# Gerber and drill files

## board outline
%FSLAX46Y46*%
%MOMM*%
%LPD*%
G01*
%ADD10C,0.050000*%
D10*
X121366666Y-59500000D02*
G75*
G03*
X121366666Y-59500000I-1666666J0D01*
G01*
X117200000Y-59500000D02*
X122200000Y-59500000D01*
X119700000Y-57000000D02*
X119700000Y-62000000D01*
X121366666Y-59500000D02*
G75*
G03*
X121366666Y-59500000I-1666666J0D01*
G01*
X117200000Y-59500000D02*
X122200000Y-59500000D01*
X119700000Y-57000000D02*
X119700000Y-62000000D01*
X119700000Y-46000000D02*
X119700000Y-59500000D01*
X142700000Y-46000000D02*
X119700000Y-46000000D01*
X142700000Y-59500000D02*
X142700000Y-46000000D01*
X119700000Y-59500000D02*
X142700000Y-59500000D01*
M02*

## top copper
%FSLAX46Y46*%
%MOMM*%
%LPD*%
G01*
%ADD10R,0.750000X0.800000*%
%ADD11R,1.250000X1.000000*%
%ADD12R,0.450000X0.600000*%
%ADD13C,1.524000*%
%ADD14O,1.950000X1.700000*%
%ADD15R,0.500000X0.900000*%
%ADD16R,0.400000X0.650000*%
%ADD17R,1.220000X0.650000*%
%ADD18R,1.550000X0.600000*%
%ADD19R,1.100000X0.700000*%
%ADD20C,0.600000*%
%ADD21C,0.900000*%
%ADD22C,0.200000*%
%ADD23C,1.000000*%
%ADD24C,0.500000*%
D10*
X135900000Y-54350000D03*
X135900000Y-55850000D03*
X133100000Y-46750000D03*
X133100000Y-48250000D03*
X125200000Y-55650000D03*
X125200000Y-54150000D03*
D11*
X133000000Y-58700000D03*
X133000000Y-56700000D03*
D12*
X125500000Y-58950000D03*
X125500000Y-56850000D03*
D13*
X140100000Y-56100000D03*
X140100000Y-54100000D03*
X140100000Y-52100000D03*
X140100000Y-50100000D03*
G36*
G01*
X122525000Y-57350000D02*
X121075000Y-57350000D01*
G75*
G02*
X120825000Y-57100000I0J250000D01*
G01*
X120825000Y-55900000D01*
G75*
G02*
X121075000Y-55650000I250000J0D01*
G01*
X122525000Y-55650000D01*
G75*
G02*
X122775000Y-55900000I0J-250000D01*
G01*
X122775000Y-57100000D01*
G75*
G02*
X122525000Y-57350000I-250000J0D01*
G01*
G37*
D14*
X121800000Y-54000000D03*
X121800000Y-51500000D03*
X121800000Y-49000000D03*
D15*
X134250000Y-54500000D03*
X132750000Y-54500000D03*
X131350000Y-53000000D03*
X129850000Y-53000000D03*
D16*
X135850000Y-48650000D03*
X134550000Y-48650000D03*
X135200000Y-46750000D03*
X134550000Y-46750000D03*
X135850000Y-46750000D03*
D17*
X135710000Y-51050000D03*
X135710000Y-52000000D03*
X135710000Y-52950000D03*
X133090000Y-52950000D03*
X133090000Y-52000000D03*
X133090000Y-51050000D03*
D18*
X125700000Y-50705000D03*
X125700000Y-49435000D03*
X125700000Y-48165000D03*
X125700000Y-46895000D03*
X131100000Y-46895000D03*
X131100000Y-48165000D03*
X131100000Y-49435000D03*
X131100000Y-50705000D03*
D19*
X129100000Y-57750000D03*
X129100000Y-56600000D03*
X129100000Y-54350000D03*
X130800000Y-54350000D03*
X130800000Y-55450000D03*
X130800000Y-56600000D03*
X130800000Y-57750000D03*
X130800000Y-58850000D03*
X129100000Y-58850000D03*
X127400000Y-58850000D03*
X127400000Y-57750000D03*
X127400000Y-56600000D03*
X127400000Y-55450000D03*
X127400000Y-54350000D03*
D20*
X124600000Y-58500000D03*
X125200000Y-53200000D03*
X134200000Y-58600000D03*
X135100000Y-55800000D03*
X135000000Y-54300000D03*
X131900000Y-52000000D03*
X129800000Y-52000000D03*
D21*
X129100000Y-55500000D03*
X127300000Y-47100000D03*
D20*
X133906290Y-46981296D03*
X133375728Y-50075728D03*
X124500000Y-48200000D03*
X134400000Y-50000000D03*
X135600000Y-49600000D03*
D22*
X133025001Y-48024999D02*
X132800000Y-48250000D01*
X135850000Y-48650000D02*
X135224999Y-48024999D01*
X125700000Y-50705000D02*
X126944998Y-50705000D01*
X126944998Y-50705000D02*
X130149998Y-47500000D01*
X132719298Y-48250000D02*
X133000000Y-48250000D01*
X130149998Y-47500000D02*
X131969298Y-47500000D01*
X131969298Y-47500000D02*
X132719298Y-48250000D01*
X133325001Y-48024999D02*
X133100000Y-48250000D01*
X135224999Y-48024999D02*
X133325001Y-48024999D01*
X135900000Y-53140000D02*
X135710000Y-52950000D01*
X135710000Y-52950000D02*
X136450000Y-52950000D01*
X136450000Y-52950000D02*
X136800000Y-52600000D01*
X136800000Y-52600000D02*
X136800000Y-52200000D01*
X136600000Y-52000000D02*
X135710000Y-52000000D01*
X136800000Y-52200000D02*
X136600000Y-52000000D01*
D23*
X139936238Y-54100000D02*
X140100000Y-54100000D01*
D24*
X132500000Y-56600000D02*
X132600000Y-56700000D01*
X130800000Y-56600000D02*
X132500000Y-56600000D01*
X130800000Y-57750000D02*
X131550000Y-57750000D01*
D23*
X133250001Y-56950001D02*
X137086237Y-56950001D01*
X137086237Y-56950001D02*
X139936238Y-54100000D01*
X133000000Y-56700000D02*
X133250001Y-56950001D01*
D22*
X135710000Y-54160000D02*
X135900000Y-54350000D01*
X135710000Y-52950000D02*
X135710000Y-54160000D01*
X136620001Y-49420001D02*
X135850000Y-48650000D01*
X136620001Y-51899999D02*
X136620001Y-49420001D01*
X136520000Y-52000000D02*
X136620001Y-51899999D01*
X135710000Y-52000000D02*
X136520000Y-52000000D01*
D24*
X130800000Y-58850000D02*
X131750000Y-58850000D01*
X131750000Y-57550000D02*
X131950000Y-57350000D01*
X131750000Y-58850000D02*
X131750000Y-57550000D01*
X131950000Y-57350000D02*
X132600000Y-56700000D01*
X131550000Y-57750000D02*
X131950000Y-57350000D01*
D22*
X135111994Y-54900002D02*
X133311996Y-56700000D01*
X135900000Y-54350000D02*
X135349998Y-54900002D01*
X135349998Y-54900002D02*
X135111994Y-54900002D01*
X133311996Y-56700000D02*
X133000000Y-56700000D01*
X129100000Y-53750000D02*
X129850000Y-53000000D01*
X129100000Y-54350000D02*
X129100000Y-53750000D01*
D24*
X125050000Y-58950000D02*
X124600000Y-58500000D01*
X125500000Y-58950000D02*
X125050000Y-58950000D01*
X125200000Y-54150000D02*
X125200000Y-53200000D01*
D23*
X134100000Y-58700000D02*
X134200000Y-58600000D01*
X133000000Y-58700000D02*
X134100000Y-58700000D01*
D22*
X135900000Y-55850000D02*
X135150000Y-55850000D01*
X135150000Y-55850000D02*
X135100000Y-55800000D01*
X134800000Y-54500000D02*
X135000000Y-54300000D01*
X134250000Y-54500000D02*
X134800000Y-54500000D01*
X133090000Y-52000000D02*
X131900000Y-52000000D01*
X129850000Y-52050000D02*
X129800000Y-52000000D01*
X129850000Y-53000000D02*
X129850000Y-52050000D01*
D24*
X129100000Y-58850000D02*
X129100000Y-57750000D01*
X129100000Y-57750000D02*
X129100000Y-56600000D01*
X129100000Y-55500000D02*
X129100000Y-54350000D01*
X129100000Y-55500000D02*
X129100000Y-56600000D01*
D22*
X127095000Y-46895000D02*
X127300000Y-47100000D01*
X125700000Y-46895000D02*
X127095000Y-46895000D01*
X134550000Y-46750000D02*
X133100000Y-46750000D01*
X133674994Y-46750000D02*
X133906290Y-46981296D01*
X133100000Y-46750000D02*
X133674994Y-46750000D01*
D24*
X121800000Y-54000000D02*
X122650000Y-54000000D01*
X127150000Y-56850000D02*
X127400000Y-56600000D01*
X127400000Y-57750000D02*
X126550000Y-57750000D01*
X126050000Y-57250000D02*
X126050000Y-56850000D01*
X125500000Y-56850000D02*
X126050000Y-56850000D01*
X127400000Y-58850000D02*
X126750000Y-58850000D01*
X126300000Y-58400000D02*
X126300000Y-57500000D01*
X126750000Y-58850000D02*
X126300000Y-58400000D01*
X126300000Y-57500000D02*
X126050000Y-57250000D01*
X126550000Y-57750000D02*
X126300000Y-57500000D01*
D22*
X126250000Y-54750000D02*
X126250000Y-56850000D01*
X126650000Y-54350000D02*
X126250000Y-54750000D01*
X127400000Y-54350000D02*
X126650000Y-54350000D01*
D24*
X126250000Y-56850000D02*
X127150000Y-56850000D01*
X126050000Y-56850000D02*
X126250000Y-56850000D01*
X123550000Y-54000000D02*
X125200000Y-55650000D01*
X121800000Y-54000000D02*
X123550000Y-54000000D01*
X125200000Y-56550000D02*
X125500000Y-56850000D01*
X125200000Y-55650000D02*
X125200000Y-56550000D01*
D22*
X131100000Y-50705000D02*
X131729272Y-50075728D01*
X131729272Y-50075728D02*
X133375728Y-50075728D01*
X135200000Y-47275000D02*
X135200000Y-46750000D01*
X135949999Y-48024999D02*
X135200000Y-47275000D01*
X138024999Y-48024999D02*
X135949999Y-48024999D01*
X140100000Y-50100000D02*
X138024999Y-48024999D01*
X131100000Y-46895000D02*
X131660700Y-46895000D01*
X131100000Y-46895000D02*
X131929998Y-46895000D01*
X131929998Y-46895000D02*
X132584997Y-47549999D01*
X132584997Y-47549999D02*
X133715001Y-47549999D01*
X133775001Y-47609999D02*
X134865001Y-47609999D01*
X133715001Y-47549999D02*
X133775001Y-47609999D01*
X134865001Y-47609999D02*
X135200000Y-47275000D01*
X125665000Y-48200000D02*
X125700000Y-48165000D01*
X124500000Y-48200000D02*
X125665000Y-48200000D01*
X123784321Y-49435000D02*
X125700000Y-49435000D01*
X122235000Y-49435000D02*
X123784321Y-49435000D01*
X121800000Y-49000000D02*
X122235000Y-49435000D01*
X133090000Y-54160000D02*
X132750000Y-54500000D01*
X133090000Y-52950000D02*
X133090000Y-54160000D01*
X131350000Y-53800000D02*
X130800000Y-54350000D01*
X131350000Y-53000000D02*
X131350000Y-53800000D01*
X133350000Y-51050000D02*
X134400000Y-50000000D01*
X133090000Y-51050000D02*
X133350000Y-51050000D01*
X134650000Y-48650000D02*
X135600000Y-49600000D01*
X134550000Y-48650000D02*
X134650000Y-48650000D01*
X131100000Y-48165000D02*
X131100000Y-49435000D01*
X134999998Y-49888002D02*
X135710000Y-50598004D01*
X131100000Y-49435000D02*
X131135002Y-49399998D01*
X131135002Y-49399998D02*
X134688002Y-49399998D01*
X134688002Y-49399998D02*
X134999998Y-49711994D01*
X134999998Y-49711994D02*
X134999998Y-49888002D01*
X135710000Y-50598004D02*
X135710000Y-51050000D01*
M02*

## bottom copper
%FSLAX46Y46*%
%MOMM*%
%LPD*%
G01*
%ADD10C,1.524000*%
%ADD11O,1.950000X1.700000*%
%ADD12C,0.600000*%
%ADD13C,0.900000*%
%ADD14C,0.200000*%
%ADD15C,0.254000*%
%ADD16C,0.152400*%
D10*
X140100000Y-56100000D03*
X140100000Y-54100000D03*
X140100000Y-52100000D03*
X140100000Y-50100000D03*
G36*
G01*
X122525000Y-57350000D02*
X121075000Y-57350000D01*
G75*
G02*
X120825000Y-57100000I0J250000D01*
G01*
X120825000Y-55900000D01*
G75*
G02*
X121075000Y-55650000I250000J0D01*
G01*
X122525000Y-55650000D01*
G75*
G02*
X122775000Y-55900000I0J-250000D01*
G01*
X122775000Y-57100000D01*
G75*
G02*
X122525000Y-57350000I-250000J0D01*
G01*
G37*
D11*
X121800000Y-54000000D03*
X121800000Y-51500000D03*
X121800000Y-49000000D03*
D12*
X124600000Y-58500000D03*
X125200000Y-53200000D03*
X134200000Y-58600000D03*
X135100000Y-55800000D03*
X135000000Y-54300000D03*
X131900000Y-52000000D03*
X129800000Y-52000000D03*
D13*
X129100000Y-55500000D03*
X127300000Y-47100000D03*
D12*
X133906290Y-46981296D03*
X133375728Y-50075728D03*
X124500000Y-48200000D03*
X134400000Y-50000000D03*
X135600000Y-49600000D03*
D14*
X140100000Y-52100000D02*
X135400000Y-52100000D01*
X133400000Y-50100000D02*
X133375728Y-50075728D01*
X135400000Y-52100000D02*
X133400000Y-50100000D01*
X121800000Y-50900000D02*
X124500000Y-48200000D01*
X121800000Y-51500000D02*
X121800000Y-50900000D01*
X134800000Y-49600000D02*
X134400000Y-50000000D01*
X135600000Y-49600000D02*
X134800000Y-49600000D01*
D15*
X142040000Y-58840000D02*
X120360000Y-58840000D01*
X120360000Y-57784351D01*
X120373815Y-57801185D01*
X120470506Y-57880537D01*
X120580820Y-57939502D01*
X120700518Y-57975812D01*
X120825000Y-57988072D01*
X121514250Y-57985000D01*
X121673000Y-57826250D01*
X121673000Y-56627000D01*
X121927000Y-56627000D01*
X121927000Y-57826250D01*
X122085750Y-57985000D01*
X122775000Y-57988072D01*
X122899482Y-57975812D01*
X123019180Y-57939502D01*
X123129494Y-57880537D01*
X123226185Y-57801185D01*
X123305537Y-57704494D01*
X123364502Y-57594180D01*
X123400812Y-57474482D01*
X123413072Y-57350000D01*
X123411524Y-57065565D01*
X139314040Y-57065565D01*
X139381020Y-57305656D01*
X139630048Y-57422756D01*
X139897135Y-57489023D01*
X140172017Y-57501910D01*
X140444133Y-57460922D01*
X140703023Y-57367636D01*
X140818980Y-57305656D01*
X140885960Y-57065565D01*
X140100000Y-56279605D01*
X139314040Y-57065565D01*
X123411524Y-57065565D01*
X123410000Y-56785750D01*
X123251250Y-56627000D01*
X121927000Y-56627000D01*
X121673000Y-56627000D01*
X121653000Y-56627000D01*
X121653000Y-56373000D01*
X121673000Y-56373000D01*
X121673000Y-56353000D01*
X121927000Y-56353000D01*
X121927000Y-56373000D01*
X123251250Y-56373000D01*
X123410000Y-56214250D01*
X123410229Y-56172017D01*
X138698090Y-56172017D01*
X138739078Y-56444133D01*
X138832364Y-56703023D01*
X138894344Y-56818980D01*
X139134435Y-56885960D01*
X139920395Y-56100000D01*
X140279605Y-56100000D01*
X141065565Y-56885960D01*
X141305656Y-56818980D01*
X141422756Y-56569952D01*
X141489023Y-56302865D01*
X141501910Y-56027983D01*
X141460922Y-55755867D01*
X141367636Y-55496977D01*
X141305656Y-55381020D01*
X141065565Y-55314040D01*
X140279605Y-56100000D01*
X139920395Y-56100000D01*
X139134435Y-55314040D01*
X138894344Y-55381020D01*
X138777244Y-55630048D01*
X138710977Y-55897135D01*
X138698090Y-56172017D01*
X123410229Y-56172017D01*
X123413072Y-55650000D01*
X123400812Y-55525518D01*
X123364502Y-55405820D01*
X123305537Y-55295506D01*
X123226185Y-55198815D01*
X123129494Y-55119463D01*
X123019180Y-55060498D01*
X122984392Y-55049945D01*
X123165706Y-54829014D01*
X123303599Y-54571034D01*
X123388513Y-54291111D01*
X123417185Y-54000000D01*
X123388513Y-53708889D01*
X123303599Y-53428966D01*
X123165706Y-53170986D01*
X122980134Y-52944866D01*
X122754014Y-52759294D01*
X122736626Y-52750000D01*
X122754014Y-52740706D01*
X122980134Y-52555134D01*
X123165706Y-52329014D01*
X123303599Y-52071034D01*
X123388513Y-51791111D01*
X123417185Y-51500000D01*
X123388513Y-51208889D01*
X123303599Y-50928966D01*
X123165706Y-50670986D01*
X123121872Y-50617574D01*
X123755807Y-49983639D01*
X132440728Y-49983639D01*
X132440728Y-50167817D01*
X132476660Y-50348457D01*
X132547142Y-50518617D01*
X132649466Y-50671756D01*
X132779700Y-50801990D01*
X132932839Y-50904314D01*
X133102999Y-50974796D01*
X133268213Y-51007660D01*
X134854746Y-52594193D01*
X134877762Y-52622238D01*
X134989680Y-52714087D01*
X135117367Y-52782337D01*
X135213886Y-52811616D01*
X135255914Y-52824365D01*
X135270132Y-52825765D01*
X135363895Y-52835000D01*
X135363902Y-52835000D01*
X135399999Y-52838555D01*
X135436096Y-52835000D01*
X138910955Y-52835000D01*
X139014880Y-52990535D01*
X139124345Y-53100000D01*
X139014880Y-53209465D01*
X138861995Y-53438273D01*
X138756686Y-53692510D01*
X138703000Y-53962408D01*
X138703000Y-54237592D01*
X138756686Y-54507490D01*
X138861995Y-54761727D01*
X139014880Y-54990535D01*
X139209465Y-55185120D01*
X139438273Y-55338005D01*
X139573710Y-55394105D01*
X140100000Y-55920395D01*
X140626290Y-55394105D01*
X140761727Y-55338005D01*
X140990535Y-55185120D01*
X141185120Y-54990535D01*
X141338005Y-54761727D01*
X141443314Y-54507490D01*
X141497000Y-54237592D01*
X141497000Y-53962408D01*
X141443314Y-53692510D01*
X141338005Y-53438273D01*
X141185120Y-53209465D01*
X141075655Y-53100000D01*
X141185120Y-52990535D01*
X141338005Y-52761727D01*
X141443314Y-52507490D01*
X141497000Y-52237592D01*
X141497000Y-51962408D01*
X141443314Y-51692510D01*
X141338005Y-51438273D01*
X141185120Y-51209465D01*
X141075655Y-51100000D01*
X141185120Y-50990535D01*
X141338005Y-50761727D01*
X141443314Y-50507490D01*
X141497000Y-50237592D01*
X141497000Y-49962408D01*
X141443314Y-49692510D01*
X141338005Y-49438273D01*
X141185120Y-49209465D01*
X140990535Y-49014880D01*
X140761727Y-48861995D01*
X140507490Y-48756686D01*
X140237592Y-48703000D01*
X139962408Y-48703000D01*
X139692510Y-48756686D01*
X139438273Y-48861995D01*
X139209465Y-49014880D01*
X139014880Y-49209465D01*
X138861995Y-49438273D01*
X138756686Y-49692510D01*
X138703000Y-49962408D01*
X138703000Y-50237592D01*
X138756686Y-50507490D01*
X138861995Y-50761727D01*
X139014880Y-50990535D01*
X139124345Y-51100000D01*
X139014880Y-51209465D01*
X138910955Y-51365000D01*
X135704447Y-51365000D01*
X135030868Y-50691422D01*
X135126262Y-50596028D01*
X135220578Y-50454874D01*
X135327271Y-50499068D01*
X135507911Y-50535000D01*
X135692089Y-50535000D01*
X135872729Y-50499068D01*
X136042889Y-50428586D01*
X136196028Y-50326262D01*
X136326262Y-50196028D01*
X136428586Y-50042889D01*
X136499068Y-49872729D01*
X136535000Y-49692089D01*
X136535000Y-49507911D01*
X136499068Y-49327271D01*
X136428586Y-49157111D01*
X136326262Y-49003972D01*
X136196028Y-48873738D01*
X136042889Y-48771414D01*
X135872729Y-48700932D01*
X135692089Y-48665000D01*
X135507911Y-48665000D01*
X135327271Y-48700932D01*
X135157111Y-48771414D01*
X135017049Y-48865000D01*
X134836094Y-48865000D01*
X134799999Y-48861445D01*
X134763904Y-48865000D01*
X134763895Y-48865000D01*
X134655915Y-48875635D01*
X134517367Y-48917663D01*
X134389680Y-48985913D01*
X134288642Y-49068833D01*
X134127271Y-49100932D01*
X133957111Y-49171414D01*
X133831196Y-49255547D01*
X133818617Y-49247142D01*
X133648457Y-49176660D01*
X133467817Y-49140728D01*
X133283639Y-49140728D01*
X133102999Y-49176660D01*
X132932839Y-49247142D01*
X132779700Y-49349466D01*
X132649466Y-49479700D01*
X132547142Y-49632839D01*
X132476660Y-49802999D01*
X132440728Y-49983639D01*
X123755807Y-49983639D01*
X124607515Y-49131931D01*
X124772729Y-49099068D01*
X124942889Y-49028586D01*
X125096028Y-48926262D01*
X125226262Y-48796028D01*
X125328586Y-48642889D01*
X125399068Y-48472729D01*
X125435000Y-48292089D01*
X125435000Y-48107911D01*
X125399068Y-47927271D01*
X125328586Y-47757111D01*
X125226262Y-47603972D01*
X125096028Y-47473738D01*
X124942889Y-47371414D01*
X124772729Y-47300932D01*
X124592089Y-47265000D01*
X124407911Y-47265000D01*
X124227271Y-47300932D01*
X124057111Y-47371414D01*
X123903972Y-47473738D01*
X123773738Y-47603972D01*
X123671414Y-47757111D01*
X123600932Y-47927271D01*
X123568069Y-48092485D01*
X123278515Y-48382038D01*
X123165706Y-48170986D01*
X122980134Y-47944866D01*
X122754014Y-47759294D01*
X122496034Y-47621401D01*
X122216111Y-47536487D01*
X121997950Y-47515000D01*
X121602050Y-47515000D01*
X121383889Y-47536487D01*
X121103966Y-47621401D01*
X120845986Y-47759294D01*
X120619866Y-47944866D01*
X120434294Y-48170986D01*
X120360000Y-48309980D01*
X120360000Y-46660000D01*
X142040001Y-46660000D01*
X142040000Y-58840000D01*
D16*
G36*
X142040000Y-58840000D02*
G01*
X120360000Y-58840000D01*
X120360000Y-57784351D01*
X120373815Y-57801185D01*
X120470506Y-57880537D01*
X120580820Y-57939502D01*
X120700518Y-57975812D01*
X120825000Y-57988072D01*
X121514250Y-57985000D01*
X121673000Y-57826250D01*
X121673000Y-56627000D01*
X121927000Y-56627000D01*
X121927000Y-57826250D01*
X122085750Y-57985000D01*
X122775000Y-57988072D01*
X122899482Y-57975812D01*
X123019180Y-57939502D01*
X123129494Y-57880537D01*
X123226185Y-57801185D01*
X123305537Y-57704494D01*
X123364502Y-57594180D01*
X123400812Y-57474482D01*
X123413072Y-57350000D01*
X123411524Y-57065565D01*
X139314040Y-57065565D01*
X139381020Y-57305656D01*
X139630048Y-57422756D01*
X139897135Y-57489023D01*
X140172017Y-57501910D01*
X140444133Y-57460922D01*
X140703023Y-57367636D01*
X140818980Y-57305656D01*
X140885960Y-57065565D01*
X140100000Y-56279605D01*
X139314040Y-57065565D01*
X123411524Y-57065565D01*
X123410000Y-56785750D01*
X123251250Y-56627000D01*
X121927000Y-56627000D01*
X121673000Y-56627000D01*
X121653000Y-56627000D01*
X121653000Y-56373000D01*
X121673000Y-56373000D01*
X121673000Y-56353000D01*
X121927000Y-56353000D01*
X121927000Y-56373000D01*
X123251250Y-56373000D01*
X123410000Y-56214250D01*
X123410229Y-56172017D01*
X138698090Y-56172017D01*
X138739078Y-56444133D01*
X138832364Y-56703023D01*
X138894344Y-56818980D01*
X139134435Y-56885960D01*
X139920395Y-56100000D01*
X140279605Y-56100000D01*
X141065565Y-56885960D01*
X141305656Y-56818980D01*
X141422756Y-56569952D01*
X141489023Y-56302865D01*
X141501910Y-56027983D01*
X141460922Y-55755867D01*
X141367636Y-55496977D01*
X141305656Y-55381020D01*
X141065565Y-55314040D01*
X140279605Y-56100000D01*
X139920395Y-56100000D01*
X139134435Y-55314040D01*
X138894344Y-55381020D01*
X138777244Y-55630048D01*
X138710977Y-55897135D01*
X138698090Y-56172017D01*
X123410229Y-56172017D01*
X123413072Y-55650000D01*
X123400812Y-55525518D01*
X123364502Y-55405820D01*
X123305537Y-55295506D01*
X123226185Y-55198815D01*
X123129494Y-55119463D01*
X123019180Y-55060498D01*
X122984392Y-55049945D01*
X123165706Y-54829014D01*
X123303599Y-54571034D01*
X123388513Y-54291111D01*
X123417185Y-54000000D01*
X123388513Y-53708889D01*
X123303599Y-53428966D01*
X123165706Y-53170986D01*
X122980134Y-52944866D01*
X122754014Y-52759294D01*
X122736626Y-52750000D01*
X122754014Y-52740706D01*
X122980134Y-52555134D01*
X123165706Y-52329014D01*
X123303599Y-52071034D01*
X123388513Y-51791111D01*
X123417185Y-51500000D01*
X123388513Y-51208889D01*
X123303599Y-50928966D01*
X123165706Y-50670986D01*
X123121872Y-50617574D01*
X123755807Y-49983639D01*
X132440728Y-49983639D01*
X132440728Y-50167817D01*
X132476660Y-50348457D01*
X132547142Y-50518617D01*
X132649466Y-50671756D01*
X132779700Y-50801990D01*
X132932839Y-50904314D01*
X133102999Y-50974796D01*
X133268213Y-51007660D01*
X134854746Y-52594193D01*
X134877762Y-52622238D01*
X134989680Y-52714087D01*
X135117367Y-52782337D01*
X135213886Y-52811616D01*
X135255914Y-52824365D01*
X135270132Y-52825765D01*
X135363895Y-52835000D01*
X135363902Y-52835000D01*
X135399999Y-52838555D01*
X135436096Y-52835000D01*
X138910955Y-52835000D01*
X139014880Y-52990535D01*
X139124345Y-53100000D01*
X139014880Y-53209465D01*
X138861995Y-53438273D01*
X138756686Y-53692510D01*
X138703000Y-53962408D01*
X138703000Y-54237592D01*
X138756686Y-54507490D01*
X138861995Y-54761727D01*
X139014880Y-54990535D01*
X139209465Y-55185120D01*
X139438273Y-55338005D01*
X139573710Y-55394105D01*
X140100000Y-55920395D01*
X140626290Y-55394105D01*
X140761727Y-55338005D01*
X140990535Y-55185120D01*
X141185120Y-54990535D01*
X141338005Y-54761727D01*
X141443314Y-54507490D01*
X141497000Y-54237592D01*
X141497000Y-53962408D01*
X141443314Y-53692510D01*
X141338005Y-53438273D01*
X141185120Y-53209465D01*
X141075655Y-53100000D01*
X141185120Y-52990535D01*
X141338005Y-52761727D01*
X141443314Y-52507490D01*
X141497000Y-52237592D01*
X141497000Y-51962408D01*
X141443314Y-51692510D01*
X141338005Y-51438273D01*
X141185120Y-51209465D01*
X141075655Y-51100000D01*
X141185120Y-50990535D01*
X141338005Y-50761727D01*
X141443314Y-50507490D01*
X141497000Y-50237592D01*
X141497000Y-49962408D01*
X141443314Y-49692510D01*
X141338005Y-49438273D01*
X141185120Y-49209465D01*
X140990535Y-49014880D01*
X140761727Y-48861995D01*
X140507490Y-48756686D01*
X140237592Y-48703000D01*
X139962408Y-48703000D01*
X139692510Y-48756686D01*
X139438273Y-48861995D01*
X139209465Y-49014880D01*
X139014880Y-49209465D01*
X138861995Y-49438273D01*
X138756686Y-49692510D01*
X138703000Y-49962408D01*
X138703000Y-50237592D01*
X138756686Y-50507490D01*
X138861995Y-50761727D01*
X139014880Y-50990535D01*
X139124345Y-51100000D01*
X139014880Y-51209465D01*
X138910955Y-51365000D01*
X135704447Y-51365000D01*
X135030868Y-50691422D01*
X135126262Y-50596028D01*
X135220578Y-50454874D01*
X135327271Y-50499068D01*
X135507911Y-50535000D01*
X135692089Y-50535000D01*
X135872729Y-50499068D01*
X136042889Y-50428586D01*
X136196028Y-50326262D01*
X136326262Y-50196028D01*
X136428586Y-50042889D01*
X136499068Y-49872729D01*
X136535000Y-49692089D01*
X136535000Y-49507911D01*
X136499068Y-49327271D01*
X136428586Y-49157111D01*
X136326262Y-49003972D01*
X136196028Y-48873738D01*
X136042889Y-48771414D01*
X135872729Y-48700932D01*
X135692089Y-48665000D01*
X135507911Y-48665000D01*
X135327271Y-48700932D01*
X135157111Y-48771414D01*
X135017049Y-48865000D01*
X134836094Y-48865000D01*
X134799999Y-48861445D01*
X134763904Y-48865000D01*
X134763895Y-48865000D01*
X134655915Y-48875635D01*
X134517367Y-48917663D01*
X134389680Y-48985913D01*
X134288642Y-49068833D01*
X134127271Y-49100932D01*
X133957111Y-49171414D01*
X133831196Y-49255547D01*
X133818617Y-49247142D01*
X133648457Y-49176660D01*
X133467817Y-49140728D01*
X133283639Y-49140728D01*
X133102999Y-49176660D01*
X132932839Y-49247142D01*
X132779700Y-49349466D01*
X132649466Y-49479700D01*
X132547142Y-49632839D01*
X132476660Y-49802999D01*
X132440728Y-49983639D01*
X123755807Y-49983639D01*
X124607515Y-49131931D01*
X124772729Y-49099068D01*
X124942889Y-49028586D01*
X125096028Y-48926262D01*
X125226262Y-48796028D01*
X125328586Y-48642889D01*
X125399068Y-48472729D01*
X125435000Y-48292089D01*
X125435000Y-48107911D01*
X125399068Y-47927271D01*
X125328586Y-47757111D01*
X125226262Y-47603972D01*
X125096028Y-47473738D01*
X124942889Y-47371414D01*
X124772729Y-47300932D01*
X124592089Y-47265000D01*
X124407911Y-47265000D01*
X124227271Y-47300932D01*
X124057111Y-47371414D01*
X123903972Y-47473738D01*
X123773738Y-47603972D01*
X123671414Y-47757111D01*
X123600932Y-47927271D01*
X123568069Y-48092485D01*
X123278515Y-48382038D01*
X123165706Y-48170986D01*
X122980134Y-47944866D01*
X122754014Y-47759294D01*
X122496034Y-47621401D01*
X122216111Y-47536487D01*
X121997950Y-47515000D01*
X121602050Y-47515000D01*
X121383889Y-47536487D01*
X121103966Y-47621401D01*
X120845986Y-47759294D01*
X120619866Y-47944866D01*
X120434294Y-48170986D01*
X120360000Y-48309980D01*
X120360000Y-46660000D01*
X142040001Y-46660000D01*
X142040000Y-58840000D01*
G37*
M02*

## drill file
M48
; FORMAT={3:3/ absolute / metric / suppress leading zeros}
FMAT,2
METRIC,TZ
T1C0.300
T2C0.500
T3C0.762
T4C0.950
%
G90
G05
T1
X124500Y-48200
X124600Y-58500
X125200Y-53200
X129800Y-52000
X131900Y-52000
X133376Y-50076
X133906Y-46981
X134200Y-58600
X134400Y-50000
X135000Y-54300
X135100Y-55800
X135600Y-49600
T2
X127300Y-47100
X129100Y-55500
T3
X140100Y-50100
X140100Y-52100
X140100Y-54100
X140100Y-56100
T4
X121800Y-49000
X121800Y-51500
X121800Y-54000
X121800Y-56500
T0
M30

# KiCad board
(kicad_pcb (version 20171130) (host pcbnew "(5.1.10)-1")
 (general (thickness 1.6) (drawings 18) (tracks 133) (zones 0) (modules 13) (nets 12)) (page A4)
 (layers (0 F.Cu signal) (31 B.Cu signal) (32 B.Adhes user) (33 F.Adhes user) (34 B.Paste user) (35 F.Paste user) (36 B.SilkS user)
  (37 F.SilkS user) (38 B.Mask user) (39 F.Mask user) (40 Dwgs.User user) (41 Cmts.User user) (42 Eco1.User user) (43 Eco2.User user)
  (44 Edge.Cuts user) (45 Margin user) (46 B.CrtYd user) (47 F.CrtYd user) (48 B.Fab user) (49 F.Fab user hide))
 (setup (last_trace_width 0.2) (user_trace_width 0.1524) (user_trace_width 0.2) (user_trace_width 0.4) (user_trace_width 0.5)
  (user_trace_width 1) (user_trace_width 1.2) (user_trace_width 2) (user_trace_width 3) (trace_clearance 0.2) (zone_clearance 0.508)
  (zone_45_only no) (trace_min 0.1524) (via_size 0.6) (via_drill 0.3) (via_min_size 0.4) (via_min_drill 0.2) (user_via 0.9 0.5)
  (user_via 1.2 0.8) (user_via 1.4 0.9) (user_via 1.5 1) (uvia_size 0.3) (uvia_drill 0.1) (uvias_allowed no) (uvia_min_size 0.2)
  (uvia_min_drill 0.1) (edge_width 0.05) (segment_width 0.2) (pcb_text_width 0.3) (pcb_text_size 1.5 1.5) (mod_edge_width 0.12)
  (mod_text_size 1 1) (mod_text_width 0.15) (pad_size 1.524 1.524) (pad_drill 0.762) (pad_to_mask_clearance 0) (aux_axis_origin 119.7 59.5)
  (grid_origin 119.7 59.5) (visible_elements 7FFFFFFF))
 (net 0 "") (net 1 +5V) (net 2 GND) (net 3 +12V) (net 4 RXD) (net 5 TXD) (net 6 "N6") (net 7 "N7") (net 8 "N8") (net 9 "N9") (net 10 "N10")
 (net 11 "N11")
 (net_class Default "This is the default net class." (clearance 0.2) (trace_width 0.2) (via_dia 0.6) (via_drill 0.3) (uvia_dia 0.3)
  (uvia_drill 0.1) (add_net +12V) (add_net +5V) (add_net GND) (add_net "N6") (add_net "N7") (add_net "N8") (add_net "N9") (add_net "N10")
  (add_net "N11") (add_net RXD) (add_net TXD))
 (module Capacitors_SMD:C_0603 (layer F.Cu) (at 135.9 55.1 270)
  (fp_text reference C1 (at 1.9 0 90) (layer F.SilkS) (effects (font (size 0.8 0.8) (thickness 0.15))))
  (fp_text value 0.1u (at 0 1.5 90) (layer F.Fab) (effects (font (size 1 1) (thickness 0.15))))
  (pad 1 smd rect (at -0.75 0 270) (size 0.8 0.75) (layers F.Cu F.Paste F.Mask) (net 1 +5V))
  (pad 2 smd rect (at 0.75 0 270) (size 0.8 0.75) (layers F.Cu F.Paste F.Mask) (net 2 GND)))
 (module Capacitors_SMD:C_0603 (layer F.Cu) (at 133.1 47.5 90)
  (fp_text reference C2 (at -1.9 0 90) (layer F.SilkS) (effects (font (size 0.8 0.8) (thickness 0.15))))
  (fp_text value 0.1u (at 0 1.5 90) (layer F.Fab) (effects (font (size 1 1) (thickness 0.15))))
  (pad 2 smd rect (at 0.75 0 90) (size 0.8 0.75) (layers F.Cu F.Paste F.Mask) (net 2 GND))
  (pad 1 smd rect (at -0.75 0 90) (size 0.8 0.75) (layers F.Cu F.Paste F.Mask) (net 1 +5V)))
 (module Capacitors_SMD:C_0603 (layer F.Cu) (at 125.2 54.9 90)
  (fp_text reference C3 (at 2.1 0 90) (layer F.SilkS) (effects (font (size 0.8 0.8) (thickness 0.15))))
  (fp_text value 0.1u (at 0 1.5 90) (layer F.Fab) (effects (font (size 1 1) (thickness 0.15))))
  (pad 1 smd rect (at -0.75 0 90) (size 0.8 0.75) (layers F.Cu F.Paste F.Mask) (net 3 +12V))
  (pad 2 smd rect (at 0.75 0 90) (size 0.8 0.75) (layers F.Cu F.Paste F.Mask) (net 2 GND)))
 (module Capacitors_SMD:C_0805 (layer F.Cu) (at 133 57.7 270)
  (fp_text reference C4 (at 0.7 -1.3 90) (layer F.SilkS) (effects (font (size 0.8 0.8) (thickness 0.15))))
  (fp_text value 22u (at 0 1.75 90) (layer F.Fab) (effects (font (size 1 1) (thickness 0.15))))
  (pad 2 smd rect (at 1 0 270) (size 1 1.25) (layers F.Cu F.Paste F.Mask) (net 2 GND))
  (pad 1 smd rect (at -1 0 270) (size 1 1.25) (layers F.Cu F.Paste F.Mask) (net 1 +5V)))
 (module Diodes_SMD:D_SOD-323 (layer F.Cu) (at 125.5 57.9 270)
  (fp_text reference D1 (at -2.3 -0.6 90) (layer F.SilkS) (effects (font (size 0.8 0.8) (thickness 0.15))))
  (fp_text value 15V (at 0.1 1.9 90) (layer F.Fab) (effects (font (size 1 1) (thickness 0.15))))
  (pad 2 smd rect (at 1.05 0 270) (size 0.6 0.45) (layers F.Cu F.Paste F.Mask) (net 2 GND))
  (pad 1 smd rect (at -1.05 0 270) (size 0.6 0.45) (layers F.Cu F.Paste F.Mask) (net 3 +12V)))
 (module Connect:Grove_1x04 (layer F.Cu) (at 140.1 50.1)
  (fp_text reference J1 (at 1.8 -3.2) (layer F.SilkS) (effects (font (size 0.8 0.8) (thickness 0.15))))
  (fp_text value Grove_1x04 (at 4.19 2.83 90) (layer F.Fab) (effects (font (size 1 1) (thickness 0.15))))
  (pad 4 thru_hole circle (at 0 6) (size 1.524 1.524) (drill 0.762) (layers *.Cu *.Mask F.SilkS) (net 2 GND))
  (pad 3 thru_hole circle (at 0 4) (size 1.524 1.524) (drill 0.762) (layers *.Cu *.Mask F.SilkS) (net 1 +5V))
  (pad 2 thru_hole circle (at 0 2) (size 1.524 1.524) (drill 0.762) (layers *.Cu *.Mask F.SilkS) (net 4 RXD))
  (pad 1 thru_hole circle (at 0 0) (size 1.524 1.524) (drill 0.762) (layers *.Cu *.Mask F.SilkS) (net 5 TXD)))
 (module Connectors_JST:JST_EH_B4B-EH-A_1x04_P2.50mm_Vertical (layer F.Cu) (at 121.8 56.5 90)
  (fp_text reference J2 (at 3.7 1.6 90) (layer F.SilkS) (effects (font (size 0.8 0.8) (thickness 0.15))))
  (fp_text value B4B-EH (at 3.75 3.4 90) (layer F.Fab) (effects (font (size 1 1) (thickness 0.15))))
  (pad 1 thru_hole roundrect (at 0 0 90) (size 1.7 1.95) (drill 0.95) (layers *.Cu *.Mask) (roundrect_rratio 0.1470588235294118) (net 2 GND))
  (pad 2 thru_hole oval (at 2.5 0 90) (size 1.7 1.95) (drill 0.95) (layers *.Cu *.Mask) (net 3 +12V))
  (pad 3 thru_hole oval (at 5 0 90) (size 1.7 1.95) (drill 0.95) (layers *.Cu *.Mask) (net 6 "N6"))
  (pad 4 thru_hole oval (at 7.5 0 90) (size 1.7 1.95) (drill 0.95) (layers *.Cu *.Mask) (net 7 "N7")))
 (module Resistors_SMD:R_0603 (layer F.Cu) (at 133.5 54.5)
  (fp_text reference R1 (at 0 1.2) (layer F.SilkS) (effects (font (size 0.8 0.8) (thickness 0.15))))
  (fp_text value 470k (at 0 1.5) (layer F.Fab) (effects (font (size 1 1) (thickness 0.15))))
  (pad 2 smd rect (at 0.75 0) (size 0.5 0.9) (layers F.Cu F.Paste F.Mask) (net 2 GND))
  (pad 1 smd rect (at -0.75 0) (size 0.5 0.9) (layers F.Cu F.Paste F.Mask) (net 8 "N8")))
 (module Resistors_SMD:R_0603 (layer F.Cu) (at 130.6 53 180)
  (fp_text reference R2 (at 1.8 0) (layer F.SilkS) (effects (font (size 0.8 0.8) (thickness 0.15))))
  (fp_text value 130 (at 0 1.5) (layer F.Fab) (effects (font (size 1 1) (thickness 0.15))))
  (pad 1 smd rect (at -0.75 0 180) (size 0.5 0.9) (layers F.Cu F.Paste F.Mask) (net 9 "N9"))
  (pad 2 smd rect (at 0.75 0 180) (size 0.5 0.9) (layers F.Cu F.Paste F.Mask) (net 2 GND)))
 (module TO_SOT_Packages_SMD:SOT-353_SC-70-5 (layer F.Cu) (at 135.2 47.7 270)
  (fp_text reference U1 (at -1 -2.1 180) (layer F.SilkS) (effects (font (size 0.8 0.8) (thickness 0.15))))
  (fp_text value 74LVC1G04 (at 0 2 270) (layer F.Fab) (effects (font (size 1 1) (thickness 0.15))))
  (pad 5 smd rect (at 0.95 -0.65 270) (size 0.65 0.4) (layers F.Cu F.Paste F.Mask) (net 1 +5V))
  (pad 4 smd rect (at 0.95 0.65 270) (size 0.65 0.4) (layers F.Cu F.Paste F.Mask) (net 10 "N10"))
  (pad 2 smd rect (at -0.95 0 270) (size 0.65 0.4) (layers F.Cu F.Paste F.Mask) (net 5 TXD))
  (pad 3 smd rect (at -0.95 0.65 270) (size 0.65 0.4) (layers F.Cu F.Paste F.Mask) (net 2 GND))
  (pad 1 smd rect (at -0.95 -0.65 270) (size 0.65 0.4) (layers F.Cu F.Paste F.Mask)))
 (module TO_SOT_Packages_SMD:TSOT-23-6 (layer F.Cu) (at 134.4 52)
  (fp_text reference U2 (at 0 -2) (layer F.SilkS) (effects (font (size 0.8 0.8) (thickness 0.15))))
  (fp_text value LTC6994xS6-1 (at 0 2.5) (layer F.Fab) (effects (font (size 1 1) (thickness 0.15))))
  (pad 6 smd rect (at 1.31 -0.95) (size 1.22 0.65) (layers F.Cu F.Paste F.Mask) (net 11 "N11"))
  (pad 5 smd rect (at 1.31 0) (size 1.22 0.65) (layers F.Cu F.Paste F.Mask) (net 1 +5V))
  (pad 4 smd rect (at 1.31 0.95) (size 1.22 0.65) (layers F.Cu F.Paste F.Mask) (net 1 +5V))
  (pad 3 smd rect (at -1.31 0.95) (size 1.22 0.65) (layers F.Cu F.Paste F.Mask) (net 8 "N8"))
  (pad 2 smd rect (at -1.31 0) (size 1.22 0.65) (layers F.Cu F.Paste F.Mask) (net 2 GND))
  (pad 1 smd rect (at -1.31 -0.95) (size 1.22 0.65) (layers F.Cu F.Paste F.Mask) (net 10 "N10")))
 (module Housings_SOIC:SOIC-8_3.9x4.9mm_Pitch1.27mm (layer F.Cu) (at 128.4 48.8 180)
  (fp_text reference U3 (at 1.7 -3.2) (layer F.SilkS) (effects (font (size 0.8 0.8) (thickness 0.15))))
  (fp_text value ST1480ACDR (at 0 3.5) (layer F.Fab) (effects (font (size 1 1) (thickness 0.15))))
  (pad 8 smd rect (at 2.7 -1.905 180) (size 1.55 0.6) (layers F.Cu F.Paste F.Mask) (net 1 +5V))
  (pad 7 smd rect (at 2.7 -0.635 180) (size 1.55 0.6) (layers F.Cu F.Paste F.Mask) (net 7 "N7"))
  (pad 6 smd rect (at 2.7 0.635 180) (size 1.55 0.6) (layers F.Cu F.Paste F.Mask) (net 6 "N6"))
  (pad 5 smd rect (at 2.7 1.905 180) (size 1.55 0.6) (layers F.Cu F.Paste F.Mask) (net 2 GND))
  (pad 4 smd rect (at -2.7 1.905 180) (size 1.55 0.6) (layers F.Cu F.Paste F.Mask) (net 5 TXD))
  (pad 3 smd rect (at -2.7 0.635 180) (size 1.55 0.6) (layers F.Cu F.Paste F.Mask) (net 11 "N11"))
  (pad 2 smd rect (at -2.7 -0.635 180) (size 1.55 0.6) (layers F.Cu F.Paste F.Mask) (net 11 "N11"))
  (pad 1 smd rect (at -2.7 -1.905 180) (size 1.55 0.6) (layers F.Cu F.Paste F.Mask) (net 4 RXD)))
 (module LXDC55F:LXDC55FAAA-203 (layer F.Cu) (at 129.1 56.6 90)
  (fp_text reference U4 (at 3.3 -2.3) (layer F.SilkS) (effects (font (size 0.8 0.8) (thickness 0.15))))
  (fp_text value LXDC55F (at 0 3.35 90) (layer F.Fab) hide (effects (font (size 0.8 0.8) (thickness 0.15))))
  (pad 14 smd rect (at -1.15 0 90) (size 0.7 1.1) (layers F.Cu F.Paste F.Mask) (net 2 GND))
  (pad 13 smd rect (at 0 0 90) (size 0.7 1.1) (layers F.Cu F.Paste F.Mask) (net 2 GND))
  (pad 12 smd rect (at 2.25 0 90) (size 0.7 1.1) (layers F.Cu F.Paste F.Mask) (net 2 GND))
  (pad 11 smd rect (at 2.25 1.7 90) (size 0.7 1.1) (layers F.Cu F.Paste F.Mask) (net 9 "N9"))
  (pad 10 smd rect (at 1.15 1.7 90) (size 0.7 1.1) (layers F.Cu F.Paste F.Mask))
  (pad 9 smd rect (at 0 1.7 90) (size 0.7 1.1) (layers F.Cu F.Paste F.Mask) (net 1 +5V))
  (pad 8 smd rect (at -1.15 1.7 90) (size 0.7 1.1) (layers F.Cu F.Paste F.Mask) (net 1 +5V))
  (pad 7 smd rect (at -2.25 1.7 90) (size 0.7 1.1) (layers F.Cu F.Paste F.Mask) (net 1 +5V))
  (pad 6 smd rect (at -2.25 0 90) (size 0.7 1.1) (layers F.Cu F.Paste F.Mask) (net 2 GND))
  (pad 5 smd rect (at -2.25 -1.7 90) (size 0.7 1.1) (layers F.Cu F.Paste F.Mask) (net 3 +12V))
  (pad 4 smd rect (at -1.15 -1.7 90) (size 0.7 1.1) (layers F.Cu F.Paste F.Mask) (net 3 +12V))
  (pad 3 smd rect (at 0 -1.7 90) (size 0.7 1.1) (layers F.Cu F.Paste F.Mask) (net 3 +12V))
  (pad 2 smd rect (at 1.15 -1.7 90) (size 0.7 1.1) (layers F.Cu F.Paste F.Mask))
  (pad 1 smd rect (at 2.25 -1.7 90) (size 0.7 1.1) (layers F.Cu F.Paste F.Mask) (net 3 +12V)))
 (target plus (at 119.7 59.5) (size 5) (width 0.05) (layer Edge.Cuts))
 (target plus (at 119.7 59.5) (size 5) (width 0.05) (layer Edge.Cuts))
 (gr_line (start 119.7 46) (end 119.7 59.5) (layer Edge.Cuts) (width 0.05))
 (gr_line (start 142.7 46) (end 119.7 46) (layer Edge.Cuts) (width 0.05))
 (gr_line (start 142.7 59.5) (end 142.7 46) (layer Edge.Cuts) (width 0.05))
 (gr_line (start 119.7 59.5) (end 142.7 59.5) (layer Edge.Cuts) (width 0.05))
 (segment (start 133.025001 48.024999) (end 132.8 48.25) (width 0.2) (layer F.Cu) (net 1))
 (segment (start 135.85 48.65) (end 135.224999 48.024999) (width 0.2) (layer F.Cu) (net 1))
 (segment (start 125.7 50.705) (end 126.944998 50.705) (width 0.2) (layer F.Cu) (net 1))
 (segment (start 126.944998 50.705) (end 130.149998 47.5) (width 0.2) (layer F.Cu) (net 1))
 (segment (start 132.719298 48.25) (end 133 48.25) (width 0.2) (layer F.Cu) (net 1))
 (segment (start 130.149998 47.5) (end 131.969298 47.5) (width 0.2) (layer F.Cu) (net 1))
 (segment (start 131.969298 47.5) (end 132.719298 48.25) (width 0.2) (layer F.Cu) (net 1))
 (segment (start 133.325001 48.024999) (end 133.1 48.25) (width 0.2) (layer F.Cu) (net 1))
 (segment (start 135.224999 48.024999) (end 133.325001 48.024999) (width 0.2) (layer F.Cu) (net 1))
 (segment (start 135.9 53.14) (end 135.71 52.95) (width 0.2) (layer F.Cu) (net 1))
 (segment (start 135.71 52.95) (end 136.45 52.95) (width 0.2) (layer F.Cu) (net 1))
 (segment (start 136.45 52.95) (end 136.8 52.6) (width 0.2) (layer F.Cu) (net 1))
 (segment (start 136.8 52.6) (end 136.8 52.2) (width 0.2) (layer F.Cu) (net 1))
 (segment (start 136.6 52) (end 135.71 52) (width 0.2) (layer F.Cu) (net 1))
 (segment (start 136.8 52.2) (end 136.6 52) (width 0.2) (layer F.Cu) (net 1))
 (segment (start 139.936238 54.1) (end 140.1 54.1) (width 1) (layer F.Cu) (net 1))
 (segment (start 132.5 56.6) (end 132.6 56.7) (width 0.5) (layer F.Cu) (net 1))
 (segment (start 130.8 56.6) (end 132.5 56.6) (width 0.5) (layer F.Cu) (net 1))
 (segment (start 130.8 57.75) (end 131.55 57.75) (width 0.5) (layer F.Cu) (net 1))
 (segment (start 133.250001 56.950001) (end 137.086237 56.950001) (width 1) (layer F.Cu) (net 1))
 (segment (start 137.086237 56.950001) (end 139.936238 54.1) (width 1) (layer F.Cu) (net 1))
 (segment (start 133 56.7) (end 133.250001 56.950001) (width 1) (layer F.Cu) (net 1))
 (segment (start 135.71 54.16) (end 135.9 54.35) (width 0.2) (layer F.Cu) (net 1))
 (segment (start 135.71 52.95) (end 135.71 54.16) (width 0.2) (layer F.Cu) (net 1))
 (segment (start 136.620001 49.420001) (end 135.85 48.65) (width 0.2) (layer F.Cu) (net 1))
 (segment (start 136.620001 51.899999) (end 136.620001 49.420001) (width 0.2) (layer F.Cu) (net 1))
 (segment (start 136.52 52) (end 136.620001 51.899999) (width 0.2) (layer F.Cu) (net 1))
 (segment (start 135.71 52) (end 136.52 52) (width 0.2) (layer F.Cu) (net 1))
 (segment (start 130.8 58.85) (end 131.75 58.85) (width 0.5) (layer F.Cu) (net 1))
 (segment (start 131.75 57.55) (end 131.95 57.35) (width 0.5) (layer F.Cu) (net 1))
 (segment (start 131.75 58.85) (end 131.75 57.55) (width 0.5) (layer F.Cu) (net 1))
 (segment (start 131.95 57.35) (end 132.6 56.7) (width 0.5) (layer F.Cu) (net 1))
 (segment (start 131.55 57.75) (end 131.95 57.35) (width 0.5) (layer F.Cu) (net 1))
 (segment (start 135.111994 54.900002) (end 133.311996 56.7) (width 0.2) (layer F.Cu) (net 1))
 (segment (start 135.9 54.35) (end 135.349998 54.900002) (width 0.2) (layer F.Cu) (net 1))
 (segment (start 135.349998 54.900002) (end 135.111994 54.900002) (width 0.2) (layer F.Cu) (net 1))
 (segment (start 133.311996 56.7) (end 133 56.7) (width 0.2) (layer F.Cu) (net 1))
 (segment (start 129.1 53.75) (end 129.85 53) (width 0.2) (layer F.Cu) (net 2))
 (segment (start 129.1 54.35) (end 129.1 53.75) (width 0.2) (layer F.Cu) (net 2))
 (via (at 124.6 58.5) (size 0.6) (drill 0.3) (layers F.Cu B.Cu) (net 2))
 (segment (start 125.05 58.95) (end 124.6 58.5) (width 0.5) (layer F.Cu) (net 2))
 (segment (start 125.5 58.95) (end 125.05 58.95) (width 0.5) (layer F.Cu) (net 2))
 (via (at 125.2 53.2) (size 0.6) (drill 0.3) (layers F.Cu B.Cu) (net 2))
 (segment (start 125.2 54.15) (end 125.2 53.2) (width 0.5) (layer F.Cu) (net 2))
 (via (at 134.2 58.6) (size 0.6) (drill 0.3) (layers F.Cu B.Cu) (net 2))
 (segment (start 134.1 58.7) (end 134.2 58.6) (width 1) (layer F.Cu) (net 2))
 (segment (start 133 58.7) (end 134.1 58.7) (width 1) (layer F.Cu) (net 2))
 (via (at 135.1 55.8) (size 0.6) (drill 0.3) (layers F.Cu B.Cu) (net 2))
 (segment (start 135.9 55.85) (end 135.15 55.85) (width 0.2) (layer F.Cu) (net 2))
 (segment (start 135.15 55.85) (end 135.1 55.8) (width 0.2) (layer F.Cu) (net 2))
 (segment (start 134.8 54.5) (end 135 54.3) (width 0.2) (layer F.Cu) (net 2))
 (segment (start 134.25 54.5) (end 134.8 54.5) (width 0.2) (layer F.Cu) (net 2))
 (via (at 135 54.3) (size 0.6) (drill 0.3) (layers F.Cu B.Cu) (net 2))
 (via (at 131.9 52) (size 0.6) (drill 0.3) (layers F.Cu B.Cu) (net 2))
 (segment (start 133.09 52) (end 131.9 52) (width 0.2) (layer F.Cu) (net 2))
 (via (at 129.8 52) (size 0.6) (drill 0.3) (layers F.Cu B.Cu) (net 2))
 (segment (start 129.85 52.05) (end 129.8 52) (width 0.2) (layer F.Cu) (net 2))
 (segment (start 129.85 53) (end 129.85 52.05) (width 0.2) (layer F.Cu) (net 2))
 (segment (start 129.1 58.85) (end 129.1 57.75) (width 0.5) (layer F.Cu) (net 2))
 (segment (start 129.1 57.75) (end 129.1 56.6) (width 0.5) (layer F.Cu) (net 2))
 (via (at 129.1 55.5) (size 0.9) (drill 0.5) (layers F.Cu B.Cu) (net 2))
 (segment (start 129.1 55.5) (end 129.1 54.35) (width 0.5) (layer F.Cu) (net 2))
 (segment (start 129.1 55.5) (end 129.1 56.6) (width 0.5) (layer F.Cu) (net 2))
 (via (at 127.3 47.1) (size 0.9) (drill 0.5) (layers F.Cu B.Cu) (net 2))
 (segment (start 127.095 46.895) (end 127.3 47.1) (width 0.2) (layer F.Cu) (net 2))
 (segment (start 125.7 46.895) (end 127.095 46.895) (width 0.2) (layer F.Cu) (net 2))
 (segment (start 134.55 46.75) (end 133.1 46.75) (width 0.2) (layer F.Cu) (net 2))
 (segment (start 133.674994 46.75) (end 133.90629 46.981296) (width 0.2) (layer F.Cu) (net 2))
 (segment (start 133.1 46.75) (end 133.674994 46.75) (width 0.2) (layer F.Cu) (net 2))
 (via (at 133.90629 46.981296) (size 0.6) (drill 0.3) (layers F.Cu B.Cu) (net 2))
 (segment (start 121.8 54) (end 122.65 54) (width 0.5) (layer F.Cu) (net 3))
 (segment (start 127.15 56.85) (end 127.4 56.6) (width 0.5) (layer F.Cu) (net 3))
 (segment (start 127.4 57.75) (end 126.55 57.75) (width 0.5) (layer F.Cu) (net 3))
 (segment (start 126.05 57.25) (end 126.05 56.85) (width 0.5) (layer F.Cu) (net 3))
 (segment (start 125.5 56.85) (end 126.05 56.85) (width 0.5) (layer F.Cu) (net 3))
 (segment (start 127.4 58.85) (end 126.75 58.85) (width 0.5) (layer F.Cu) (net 3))
 (segment (start 126.3 58.4) (end 126.3 57.5) (width 0.5) (layer F.Cu) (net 3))
 (segment (start 126.75 58.85) (end 126.3 58.4) (width 0.5) (layer F.Cu) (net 3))
 (segment (start 126.3 57.5) (end 126.05 57.25) (width 0.5) (layer F.Cu) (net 3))
 (segment (start 126.55 57.75) (end 126.3 57.5) (width 0.5) (layer F.Cu) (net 3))
 (segment (start 126.25 54.75) (end 126.25 56.85) (width 0.2) (layer F.Cu) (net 3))
 (segment (start 126.65 54.35) (end 126.25 54.75) (width 0.2) (layer F.Cu) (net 3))
 (segment (start 127.4 54.35) (end 126.65 54.35) (width 0.2) (layer F.Cu) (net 3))
 (segment (start 126.25 56.85) (end 127.15 56.85) (width 0.5) (layer F.Cu) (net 3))
 (segment (start 126.05 56.85) (end 126.25 56.85) (width 0.5) (layer F.Cu) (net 3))
 (segment (start 123.55 54) (end 125.2 55.65) (width 0.5) (layer F.Cu) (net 3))
 (segment (start 121.8 54) (end 123.55 54) (width 0.5) (layer F.Cu) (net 3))
 (segment (start 125.2 56.55) (end 125.5 56.85) (width 0.5) (layer F.Cu) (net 3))
 (segment (start 125.2 55.65) (end 125.2 56.55) (width 0.5) (layer F.Cu) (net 3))
 (segment (start 131.1 50.705) (end 131.729272 50.075728) (width 0.2) (layer F.Cu) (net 4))
 (segment (start 140.1 52.1) (end 135.4 52.1) (width 0.2) (layer B.Cu) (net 4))
 (segment (start 133.4 50.1) (end 133.375728 50.075728) (width 0.2) (layer B.Cu) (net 4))
 (segment (start 131.729272 50.075728) (end 133.375728 50.075728) (width 0.2) (layer F.Cu) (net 4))
 (via (at 133.375728 50.075728) (size 0.6) (drill 0.3) (layers F.Cu B.Cu) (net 4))
 (segment (start 135.4 52.1) (end 133.4 50.1) (width 0.2) (layer B.Cu) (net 4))
 (segment (start 135.2 47.275) (end 135.2 46.75) (width 0.2) (layer F.Cu) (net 5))
 (segment (start 135.949999 48.024999) (end 135.2 47.275) (width 0.2) (layer F.Cu) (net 5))
 (segment (start 138.024999 48.024999) (end 135.949999 48.024999) (width 0.2) (layer F.Cu) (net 5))
 (segment (start 140.1 50.1) (end 138.024999 48.024999) (width 0.2) (layer F.Cu) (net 5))
 (segment (start 131.1 46.895) (end 131.6607 46.895) (width 0.2) (layer F.Cu) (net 5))
 (segment (start 131.1 46.895) (end 131.929998 46.895) (width 0.2) (layer F.Cu) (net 5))
 (segment (start 131.929998 46.895) (end 132.584997 47.549999) (width 0.2) (layer F.Cu) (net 5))
 (segment (start 132.584997 47.549999) (end 133.715001 47.549999) (width 0.2) (layer F.Cu) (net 5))
 (segment (start 133.775001 47.609999) (end 134.865001 47.609999) (width 0.2) (layer F.Cu) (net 5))
 (segment (start 133.715001 47.549999) (end 133.775001 47.609999) (width 0.2) (layer F.Cu) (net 5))
 (segment (start 134.865001 47.609999) (end 135.2 47.275) (width 0.2) (layer F.Cu) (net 5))
 (segment (start 121.8 50.9) (end 124.5 48.2) (width 0.2) (layer B.Cu) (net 6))
 (via (at 124.5 48.2) (size 0.6) (drill 0.3) (layers F.Cu B.Cu) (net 6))
 (segment (start 121.8 51.5) (end 121.8 50.9) (width 0.2) (layer B.Cu) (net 6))
 (segment (start 125.665 48.2) (end 125.7 48.165) (width 0.2) (layer F.Cu) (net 6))
 (segment (start 124.5 48.2) (end 125.665 48.2) (width 0.2) (layer F.Cu) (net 6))
 (segment (start 123.784321 49.435) (end 125.7 49.435) (width 0.2) (layer F.Cu) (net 7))
 (segment (start 122.235 49.435) (end 123.784321 49.435) (width 0.2) (layer F.Cu) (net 7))
 (segment (start 121.8 49) (end 122.235 49.435) (width 0.2) (layer F.Cu) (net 7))
 (segment (start 133.09 54.16) (end 132.75 54.5) (width 0.2) (layer F.Cu) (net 8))
 (segment (start 133.09 52.95) (end 133.09 54.16) (width 0.2) (layer F.Cu) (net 8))
 (segment (start 131.35 53.8) (end 130.8 54.35) (width 0.2) (layer F.Cu) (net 9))
 (segment (start 131.35 53) (end 131.35 53.8) (width 0.2) (layer F.Cu) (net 9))
 (segment (start 133.35 51.05) (end 134.4 50) (width 0.2) (layer F.Cu) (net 10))
 (via (at 134.4 50) (size 0.6) (drill 0.3) (layers F.Cu B.Cu) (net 10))
 (segment (start 133.09 51.05) (end 133.35 51.05) (width 0.2) (layer F.Cu) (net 10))
 (via (at 135.6 49.6) (size 0.6) (drill 0.3) (layers F.Cu B.Cu) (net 10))
 (segment (start 134.65 48.65) (end 135.6 49.6) (width 0.2) (layer F.Cu) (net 10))
 (segment (start 134.55 48.65) (end 134.65 48.65) (width 0.2) (layer F.Cu) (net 10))
 (segment (start 134.8 49.6) (end 134.4 50) (width 0.2) (layer B.Cu) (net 10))
 (segment (start 135.6 49.6) (end 134.8 49.6) (width 0.2) (layer B.Cu) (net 10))
 (segment (start 131.1 48.165) (end 131.1 49.435) (width 0.2) (layer F.Cu) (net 11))
 (segment (start 134.999998 49.888002) (end 135.71 50.598004) (width 0.2) (layer F.Cu) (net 11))
 (segment (start 131.1 49.435) (end 131.135002 49.399998) (width 0.2) (layer F.Cu) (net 11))
 (segment (start 131.135002 49.399998) (end 134.688002 49.399998) (width 0.2) (layer F.Cu) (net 11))
 (segment (start 134.688002 49.399998) (end 134.999998 49.711994) (width 0.2) (layer F.Cu) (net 11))
 (segment (start 134.999998 49.711994) (end 134.999998 49.888002) (width 0.2) (layer F.Cu) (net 11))
 (segment (start 135.71 50.598004) (end 135.71 51.05) (width 0.2) (layer F.Cu) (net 11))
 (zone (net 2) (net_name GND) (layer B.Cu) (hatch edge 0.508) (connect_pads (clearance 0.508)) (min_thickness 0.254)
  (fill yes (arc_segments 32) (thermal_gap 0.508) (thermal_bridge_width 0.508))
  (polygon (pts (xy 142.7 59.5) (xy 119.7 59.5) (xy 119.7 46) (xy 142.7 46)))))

